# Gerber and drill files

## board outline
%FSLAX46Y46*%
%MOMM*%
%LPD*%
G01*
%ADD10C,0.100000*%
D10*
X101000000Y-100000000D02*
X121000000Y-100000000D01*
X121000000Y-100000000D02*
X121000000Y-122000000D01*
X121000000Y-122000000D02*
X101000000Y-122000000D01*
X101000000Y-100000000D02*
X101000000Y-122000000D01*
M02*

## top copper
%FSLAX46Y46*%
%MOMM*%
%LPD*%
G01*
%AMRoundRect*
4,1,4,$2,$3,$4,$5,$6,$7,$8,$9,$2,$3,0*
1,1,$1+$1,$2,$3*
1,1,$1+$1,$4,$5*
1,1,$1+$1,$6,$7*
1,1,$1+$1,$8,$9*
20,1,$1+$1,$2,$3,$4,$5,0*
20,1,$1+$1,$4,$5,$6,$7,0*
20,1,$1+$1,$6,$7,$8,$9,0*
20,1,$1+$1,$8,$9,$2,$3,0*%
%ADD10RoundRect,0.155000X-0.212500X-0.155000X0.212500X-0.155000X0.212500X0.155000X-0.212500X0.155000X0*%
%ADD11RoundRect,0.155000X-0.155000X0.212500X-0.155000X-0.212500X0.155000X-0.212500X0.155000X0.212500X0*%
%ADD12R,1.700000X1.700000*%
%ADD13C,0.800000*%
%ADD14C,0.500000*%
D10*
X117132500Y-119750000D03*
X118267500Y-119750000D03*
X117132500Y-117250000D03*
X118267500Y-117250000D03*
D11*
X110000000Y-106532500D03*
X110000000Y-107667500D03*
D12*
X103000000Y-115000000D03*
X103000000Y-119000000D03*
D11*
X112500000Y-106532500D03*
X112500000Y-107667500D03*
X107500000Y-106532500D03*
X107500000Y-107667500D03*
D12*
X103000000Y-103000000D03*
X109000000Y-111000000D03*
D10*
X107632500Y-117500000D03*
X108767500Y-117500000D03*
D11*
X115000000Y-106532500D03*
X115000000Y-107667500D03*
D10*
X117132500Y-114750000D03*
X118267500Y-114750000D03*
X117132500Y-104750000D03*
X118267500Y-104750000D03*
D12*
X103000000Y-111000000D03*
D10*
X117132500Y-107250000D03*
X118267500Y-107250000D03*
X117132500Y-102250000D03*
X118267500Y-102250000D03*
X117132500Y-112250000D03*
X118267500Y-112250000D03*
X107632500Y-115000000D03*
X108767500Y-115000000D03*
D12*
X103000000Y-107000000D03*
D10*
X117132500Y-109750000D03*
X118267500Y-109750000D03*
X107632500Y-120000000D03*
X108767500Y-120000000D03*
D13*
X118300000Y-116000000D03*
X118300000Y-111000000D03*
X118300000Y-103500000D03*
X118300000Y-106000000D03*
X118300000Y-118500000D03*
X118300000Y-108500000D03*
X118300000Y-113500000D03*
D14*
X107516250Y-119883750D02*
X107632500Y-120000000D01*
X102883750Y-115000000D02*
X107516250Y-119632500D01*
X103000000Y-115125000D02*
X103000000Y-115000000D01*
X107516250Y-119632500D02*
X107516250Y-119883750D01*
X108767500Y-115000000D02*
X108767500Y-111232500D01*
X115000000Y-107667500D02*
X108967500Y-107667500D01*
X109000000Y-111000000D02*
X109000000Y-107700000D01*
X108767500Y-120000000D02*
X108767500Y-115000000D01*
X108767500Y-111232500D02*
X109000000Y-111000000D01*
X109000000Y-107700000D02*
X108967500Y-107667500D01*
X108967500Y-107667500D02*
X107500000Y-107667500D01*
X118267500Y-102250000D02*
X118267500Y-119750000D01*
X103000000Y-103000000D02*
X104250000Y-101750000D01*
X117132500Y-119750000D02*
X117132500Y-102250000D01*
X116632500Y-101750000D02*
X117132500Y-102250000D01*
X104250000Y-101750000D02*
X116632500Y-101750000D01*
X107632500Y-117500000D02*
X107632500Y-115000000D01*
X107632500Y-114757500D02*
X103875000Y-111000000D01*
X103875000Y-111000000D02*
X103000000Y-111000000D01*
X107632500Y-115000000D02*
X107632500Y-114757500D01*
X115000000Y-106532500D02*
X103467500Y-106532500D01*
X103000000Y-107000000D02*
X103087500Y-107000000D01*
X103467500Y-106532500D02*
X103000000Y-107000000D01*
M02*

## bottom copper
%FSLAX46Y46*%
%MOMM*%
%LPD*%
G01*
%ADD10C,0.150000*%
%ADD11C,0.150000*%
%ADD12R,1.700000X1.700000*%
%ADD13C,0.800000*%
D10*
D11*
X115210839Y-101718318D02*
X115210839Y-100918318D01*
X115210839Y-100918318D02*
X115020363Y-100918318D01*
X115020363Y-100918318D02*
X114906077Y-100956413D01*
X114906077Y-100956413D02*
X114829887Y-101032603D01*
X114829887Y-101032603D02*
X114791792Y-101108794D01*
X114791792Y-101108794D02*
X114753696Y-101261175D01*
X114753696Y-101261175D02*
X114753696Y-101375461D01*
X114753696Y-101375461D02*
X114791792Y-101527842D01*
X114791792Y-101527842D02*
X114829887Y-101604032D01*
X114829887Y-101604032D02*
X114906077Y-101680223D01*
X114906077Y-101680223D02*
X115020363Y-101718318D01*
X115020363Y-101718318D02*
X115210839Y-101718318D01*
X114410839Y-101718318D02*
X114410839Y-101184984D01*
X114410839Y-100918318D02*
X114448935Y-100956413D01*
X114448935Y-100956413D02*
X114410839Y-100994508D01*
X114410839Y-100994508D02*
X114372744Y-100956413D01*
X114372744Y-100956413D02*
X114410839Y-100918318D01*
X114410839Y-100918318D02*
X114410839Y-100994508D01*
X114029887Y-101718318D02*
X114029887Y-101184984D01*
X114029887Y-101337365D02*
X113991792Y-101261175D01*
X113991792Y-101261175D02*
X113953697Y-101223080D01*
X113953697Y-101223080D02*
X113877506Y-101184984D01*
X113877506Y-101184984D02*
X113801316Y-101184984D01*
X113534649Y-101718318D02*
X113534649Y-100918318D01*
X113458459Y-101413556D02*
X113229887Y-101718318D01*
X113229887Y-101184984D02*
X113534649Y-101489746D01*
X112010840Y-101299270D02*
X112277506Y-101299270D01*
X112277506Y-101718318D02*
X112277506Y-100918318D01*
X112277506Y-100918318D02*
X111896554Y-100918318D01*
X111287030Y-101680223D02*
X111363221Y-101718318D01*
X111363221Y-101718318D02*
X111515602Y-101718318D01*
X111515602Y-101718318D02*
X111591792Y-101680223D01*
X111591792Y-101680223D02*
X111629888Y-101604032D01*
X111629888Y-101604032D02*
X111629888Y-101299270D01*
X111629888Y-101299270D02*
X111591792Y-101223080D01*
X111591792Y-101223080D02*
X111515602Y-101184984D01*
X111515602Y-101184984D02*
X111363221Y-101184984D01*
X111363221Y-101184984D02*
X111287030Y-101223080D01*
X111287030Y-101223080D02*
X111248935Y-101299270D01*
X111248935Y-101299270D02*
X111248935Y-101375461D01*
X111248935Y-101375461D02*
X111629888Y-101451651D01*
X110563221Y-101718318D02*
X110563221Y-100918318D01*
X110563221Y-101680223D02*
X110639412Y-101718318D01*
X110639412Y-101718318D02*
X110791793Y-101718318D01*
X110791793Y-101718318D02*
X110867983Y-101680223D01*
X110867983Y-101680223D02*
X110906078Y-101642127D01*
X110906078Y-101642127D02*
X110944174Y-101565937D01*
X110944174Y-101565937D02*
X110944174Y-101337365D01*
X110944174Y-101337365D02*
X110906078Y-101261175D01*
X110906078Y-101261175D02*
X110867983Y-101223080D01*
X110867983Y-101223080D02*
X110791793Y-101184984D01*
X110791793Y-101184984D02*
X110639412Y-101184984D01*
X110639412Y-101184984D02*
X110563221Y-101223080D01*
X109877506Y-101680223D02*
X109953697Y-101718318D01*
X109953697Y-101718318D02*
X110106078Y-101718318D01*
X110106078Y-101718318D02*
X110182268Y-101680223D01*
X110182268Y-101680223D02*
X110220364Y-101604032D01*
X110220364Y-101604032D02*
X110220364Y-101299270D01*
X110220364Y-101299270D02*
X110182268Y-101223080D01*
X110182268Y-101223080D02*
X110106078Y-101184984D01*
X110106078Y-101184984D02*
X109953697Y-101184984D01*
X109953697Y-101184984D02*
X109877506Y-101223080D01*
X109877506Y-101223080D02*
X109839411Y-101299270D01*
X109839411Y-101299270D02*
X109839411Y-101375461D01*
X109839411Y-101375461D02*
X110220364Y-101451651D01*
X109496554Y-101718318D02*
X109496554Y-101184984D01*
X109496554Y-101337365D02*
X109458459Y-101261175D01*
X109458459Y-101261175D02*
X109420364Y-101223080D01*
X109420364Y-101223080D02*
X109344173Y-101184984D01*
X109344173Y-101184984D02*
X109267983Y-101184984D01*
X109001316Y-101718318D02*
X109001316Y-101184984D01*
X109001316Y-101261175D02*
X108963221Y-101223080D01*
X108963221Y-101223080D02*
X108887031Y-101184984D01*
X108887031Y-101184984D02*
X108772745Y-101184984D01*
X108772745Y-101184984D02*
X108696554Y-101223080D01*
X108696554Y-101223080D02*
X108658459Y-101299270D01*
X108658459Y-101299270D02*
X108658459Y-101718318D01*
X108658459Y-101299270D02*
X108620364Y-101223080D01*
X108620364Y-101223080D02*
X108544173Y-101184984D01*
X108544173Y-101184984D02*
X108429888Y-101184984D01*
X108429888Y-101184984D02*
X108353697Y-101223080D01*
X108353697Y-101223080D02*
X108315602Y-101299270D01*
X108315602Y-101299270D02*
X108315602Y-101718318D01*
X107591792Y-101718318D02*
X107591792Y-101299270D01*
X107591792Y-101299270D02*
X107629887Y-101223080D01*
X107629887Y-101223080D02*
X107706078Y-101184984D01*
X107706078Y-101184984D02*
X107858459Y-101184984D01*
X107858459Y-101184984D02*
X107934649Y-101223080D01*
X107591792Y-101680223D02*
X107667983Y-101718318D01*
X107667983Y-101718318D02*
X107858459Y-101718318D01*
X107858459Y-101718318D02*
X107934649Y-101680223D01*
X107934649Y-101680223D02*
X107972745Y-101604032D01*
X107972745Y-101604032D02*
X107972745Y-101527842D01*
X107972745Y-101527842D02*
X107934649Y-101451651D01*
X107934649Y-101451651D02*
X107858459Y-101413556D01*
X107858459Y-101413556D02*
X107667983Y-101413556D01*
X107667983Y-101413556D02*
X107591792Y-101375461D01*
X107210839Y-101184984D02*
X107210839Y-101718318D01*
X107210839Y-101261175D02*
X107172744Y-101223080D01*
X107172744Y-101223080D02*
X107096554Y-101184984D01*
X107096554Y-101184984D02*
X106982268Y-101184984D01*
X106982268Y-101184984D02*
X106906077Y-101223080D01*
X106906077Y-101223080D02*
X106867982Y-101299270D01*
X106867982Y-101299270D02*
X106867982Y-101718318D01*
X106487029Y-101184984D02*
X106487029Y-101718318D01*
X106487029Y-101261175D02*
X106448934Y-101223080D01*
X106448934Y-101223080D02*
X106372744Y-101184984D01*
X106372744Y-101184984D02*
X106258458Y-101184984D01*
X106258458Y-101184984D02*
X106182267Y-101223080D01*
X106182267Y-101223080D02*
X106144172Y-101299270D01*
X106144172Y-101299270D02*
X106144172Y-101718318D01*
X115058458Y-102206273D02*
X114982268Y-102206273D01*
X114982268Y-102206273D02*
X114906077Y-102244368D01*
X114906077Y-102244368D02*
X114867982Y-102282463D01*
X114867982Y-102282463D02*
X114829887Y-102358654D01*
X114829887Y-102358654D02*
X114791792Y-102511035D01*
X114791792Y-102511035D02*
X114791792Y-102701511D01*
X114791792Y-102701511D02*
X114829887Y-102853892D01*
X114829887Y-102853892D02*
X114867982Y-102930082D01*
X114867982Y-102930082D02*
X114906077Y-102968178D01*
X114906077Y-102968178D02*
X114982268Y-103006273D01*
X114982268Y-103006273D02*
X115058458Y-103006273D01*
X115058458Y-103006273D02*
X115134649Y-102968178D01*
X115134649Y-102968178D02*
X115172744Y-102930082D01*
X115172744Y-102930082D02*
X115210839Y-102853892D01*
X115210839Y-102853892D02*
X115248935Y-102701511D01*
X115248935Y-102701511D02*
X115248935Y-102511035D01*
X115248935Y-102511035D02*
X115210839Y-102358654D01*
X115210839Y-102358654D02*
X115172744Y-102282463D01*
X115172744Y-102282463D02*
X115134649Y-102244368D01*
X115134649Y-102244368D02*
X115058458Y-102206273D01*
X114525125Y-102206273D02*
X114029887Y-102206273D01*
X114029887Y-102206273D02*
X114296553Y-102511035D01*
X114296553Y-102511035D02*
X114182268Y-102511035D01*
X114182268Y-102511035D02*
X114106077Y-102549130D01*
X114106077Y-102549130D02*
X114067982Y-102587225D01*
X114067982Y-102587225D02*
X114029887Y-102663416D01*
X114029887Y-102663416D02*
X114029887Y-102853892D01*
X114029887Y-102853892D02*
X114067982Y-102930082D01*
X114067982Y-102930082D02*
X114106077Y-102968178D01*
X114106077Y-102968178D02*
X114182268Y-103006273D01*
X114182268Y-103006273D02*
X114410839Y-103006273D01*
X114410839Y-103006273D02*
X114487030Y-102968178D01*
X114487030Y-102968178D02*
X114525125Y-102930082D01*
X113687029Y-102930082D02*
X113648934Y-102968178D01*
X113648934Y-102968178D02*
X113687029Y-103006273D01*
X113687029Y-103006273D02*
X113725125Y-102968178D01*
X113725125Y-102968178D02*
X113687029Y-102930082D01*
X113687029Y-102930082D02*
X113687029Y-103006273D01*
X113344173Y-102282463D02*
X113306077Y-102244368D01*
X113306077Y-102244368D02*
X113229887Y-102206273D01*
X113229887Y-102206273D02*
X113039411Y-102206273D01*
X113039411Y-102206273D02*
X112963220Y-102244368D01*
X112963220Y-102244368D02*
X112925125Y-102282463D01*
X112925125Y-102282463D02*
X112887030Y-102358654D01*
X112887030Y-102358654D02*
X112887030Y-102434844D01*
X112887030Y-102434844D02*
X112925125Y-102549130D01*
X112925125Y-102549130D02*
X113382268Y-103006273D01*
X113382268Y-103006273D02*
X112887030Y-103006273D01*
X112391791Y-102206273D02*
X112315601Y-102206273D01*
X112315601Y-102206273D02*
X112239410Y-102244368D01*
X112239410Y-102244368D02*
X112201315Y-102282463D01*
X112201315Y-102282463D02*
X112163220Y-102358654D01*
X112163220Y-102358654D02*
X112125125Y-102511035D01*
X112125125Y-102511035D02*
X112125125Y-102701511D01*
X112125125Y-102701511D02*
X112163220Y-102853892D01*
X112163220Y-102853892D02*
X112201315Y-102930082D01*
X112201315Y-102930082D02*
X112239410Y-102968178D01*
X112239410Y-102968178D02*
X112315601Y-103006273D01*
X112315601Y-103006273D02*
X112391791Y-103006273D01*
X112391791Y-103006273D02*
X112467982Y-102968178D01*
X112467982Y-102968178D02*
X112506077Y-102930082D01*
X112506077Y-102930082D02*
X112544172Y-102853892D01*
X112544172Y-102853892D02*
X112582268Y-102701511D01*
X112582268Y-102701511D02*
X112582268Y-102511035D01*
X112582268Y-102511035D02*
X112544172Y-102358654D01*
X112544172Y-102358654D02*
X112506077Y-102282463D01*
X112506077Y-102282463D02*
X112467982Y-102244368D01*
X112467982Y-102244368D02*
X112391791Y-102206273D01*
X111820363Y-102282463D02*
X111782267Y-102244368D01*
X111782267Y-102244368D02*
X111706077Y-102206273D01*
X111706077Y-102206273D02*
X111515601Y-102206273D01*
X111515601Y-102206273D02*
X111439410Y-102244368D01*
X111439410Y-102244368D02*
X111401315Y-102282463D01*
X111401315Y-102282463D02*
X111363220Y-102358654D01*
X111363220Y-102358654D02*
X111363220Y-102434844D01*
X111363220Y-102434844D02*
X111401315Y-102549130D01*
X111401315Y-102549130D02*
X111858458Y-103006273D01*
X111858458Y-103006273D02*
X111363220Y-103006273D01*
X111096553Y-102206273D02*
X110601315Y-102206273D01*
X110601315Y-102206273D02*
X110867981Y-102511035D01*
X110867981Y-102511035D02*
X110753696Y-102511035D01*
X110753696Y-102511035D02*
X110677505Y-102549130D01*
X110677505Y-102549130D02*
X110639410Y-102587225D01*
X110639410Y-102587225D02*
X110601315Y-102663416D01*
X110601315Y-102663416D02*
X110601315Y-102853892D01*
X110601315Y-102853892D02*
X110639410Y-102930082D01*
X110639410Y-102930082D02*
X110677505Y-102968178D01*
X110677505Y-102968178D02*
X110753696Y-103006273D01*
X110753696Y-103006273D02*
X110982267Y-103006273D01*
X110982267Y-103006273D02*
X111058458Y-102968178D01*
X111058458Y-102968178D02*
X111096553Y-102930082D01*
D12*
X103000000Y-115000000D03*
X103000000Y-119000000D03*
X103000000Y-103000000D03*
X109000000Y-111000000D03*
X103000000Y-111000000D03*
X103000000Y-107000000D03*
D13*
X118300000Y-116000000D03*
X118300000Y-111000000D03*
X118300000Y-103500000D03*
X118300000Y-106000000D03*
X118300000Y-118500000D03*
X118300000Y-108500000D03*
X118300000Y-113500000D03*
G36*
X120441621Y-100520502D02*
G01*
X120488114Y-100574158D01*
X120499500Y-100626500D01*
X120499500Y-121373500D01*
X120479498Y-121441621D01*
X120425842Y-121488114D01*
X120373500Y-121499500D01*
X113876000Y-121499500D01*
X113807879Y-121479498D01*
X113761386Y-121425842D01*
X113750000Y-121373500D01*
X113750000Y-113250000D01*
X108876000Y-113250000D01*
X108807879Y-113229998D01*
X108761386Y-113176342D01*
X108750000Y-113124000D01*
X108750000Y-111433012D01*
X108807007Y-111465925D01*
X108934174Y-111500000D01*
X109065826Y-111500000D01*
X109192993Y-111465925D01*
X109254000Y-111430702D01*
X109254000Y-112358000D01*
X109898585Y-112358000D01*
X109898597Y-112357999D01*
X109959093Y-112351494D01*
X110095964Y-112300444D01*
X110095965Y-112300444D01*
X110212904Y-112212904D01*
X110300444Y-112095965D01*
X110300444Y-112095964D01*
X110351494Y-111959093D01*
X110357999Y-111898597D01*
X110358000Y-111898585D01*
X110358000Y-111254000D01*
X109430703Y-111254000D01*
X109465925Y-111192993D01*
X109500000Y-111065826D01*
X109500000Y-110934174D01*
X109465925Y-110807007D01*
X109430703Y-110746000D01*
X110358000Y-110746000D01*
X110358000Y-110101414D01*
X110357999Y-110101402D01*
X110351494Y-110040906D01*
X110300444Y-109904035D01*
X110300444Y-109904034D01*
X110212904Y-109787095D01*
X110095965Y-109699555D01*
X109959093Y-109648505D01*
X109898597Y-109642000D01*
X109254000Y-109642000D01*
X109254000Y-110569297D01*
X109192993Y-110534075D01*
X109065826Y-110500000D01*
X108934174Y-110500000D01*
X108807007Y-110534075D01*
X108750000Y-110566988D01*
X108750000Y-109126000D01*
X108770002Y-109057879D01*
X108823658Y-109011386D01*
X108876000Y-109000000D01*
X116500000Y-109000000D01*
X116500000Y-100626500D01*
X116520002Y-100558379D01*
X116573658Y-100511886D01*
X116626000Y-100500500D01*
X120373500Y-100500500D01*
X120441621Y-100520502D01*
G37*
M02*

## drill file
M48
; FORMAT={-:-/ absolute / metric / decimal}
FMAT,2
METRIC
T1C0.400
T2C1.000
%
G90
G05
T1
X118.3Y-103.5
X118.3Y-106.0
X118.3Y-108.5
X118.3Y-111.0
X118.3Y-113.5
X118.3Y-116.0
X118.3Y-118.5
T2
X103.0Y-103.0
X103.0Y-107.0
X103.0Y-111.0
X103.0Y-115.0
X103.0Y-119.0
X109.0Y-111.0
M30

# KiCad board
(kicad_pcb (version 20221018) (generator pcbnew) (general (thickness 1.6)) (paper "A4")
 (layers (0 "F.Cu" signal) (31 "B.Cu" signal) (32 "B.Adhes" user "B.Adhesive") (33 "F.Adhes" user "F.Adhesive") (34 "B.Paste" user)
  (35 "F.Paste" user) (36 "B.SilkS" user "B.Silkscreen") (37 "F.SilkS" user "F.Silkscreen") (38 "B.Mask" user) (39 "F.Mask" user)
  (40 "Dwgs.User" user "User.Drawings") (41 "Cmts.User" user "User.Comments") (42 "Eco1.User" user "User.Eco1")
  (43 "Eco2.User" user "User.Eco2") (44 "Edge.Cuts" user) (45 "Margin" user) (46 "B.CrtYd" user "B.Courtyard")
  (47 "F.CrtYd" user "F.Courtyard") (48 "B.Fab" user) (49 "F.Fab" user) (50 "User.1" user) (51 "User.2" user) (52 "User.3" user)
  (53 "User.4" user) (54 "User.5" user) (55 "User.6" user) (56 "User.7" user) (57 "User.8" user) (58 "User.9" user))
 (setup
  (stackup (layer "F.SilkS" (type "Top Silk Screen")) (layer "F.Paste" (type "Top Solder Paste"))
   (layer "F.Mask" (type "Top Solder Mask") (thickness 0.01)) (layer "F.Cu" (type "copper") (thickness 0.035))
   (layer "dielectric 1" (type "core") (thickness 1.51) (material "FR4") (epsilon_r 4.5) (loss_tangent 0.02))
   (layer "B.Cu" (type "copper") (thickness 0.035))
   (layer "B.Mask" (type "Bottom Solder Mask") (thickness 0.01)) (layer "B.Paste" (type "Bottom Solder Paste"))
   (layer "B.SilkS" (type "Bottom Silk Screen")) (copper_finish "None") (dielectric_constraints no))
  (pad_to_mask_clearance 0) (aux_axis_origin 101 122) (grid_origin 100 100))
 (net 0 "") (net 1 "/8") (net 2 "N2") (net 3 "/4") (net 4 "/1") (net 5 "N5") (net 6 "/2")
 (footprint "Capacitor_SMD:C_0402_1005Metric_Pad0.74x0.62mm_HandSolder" (layer "F.Cu") (at 117.7 119.75)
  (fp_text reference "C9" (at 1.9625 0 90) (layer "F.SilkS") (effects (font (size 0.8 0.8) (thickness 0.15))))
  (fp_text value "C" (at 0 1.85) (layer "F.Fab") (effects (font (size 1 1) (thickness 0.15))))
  (pad "1" smd roundrect (at -0.5675 0) (size 0.735 0.62) (layers "F.Cu" "F.Paste" "F.Mask") (roundrect_rratio 0.25) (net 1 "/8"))
  (pad "2" smd roundrect (at 0.5675 0) (size 0.735 0.62) (layers "F.Cu" "F.Paste" "F.Mask") (roundrect_rratio 0.25) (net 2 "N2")))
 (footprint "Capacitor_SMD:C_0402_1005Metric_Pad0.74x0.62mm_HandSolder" (layer "F.Cu") (at 117.7 117.25)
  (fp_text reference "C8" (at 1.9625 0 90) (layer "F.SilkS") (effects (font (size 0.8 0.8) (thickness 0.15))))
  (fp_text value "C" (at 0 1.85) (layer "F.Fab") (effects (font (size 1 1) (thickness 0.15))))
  (pad "1" smd roundrect (at -0.5675 0) (size 0.735 0.62) (layers "F.Cu" "F.Paste" "F.Mask") (roundrect_rratio 0.25) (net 1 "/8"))
  (pad "2" smd roundrect (at 0.5675 0) (size 0.735 0.62) (layers "F.Cu" "F.Paste" "F.Mask") (roundrect_rratio 0.25) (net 2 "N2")))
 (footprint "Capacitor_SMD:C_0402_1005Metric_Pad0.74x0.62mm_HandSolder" (layer "F.Cu") (at 110 107.1 -90)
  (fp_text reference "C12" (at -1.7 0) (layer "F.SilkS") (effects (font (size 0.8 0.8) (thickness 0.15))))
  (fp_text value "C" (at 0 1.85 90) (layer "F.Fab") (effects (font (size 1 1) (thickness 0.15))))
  (pad "1" smd roundrect (at -0.5675 0 270) (size 0.735 0.62) (layers "F.Cu" "F.Paste" "F.Mask") (roundrect_rratio 0.25) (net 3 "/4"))
  (pad "2" smd roundrect (at 0.5675 0 270) (size 0.735 0.62) (layers "F.Cu" "F.Paste" "F.Mask") (roundrect_rratio 0.25) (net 2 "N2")))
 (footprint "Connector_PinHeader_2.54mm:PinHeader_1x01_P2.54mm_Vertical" (layer "F.Cu") (at 103 115)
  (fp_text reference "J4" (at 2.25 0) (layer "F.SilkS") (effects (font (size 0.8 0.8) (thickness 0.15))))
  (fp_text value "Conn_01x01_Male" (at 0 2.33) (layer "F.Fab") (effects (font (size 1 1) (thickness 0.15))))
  (pad "1" thru_hole rect (at 0 0) (size 1.7 1.7) (drill 1) (layers "*.Cu" "*.Mask") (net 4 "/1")))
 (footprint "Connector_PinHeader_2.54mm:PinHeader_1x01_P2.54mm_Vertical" (layer "F.Cu") (at 103 119)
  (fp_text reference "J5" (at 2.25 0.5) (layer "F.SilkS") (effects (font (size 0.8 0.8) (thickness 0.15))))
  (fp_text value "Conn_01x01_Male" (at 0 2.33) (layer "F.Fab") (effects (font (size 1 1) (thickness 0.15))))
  (pad "1" thru_hole rect (at 0 0) (size 1.7 1.7) (drill 1) (layers "*.Cu" "*.Mask") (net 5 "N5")))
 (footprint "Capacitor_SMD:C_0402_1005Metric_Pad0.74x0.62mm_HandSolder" (layer "F.Cu") (at 112.5 107.1 -90)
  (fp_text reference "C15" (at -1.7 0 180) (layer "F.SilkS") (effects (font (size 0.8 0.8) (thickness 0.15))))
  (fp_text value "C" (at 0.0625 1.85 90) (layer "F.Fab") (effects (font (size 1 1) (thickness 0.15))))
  (pad "1" smd roundrect (at -0.5675 0 270) (size 0.735 0.62) (layers "F.Cu" "F.Paste" "F.Mask") (roundrect_rratio 0.25) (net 3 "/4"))
  (pad "2" smd roundrect (at 0.5675 0 270) (size 0.735 0.62) (layers "F.Cu" "F.Paste" "F.Mask") (roundrect_rratio 0.25) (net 2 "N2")))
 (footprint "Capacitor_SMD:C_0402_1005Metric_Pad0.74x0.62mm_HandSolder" (layer "F.Cu") (at 107.5 107.1 -90)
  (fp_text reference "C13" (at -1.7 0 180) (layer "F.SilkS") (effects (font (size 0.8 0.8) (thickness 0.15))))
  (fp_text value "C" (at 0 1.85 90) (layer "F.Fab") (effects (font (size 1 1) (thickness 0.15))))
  (pad "1" smd roundrect (at -0.5675 0 270) (size 0.735 0.62) (layers "F.Cu" "F.Paste" "F.Mask") (roundrect_rratio 0.25) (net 3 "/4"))
  (pad "2" smd roundrect (at 0.5675 0 270) (size 0.735 0.62) (layers "F.Cu" "F.Paste" "F.Mask") (roundrect_rratio 0.25) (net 2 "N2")))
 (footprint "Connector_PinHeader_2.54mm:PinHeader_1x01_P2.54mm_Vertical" (layer "F.Cu") (at 103 103)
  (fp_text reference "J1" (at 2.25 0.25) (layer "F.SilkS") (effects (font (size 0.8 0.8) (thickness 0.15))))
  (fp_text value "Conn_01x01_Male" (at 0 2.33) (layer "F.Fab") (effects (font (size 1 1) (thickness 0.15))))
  (pad "1" thru_hole rect (at 0 0) (size 1.7 1.7) (drill 1) (layers "*.Cu" "*.Mask") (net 1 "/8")))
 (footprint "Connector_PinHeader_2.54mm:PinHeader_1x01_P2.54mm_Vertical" (layer "F.Cu") (at 109 111)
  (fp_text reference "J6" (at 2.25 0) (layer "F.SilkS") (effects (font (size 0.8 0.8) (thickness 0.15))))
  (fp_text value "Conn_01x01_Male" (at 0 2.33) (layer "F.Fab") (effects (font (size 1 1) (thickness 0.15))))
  (pad "1" thru_hole rect (at 0 0) (size 1.7 1.7) (drill 1) (layers "*.Cu" "*.Mask") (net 2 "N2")))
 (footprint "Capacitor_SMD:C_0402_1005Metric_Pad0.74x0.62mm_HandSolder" (layer "F.Cu") (at 108.2 117.5)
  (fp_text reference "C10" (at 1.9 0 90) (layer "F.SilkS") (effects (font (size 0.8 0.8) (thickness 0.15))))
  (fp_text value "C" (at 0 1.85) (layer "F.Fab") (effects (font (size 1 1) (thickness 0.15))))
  (pad "1" smd roundrect (at -0.5675 0) (size 0.735 0.62) (layers "F.Cu" "F.Paste" "F.Mask") (roundrect_rratio 0.25) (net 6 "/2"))
  (pad "2" smd roundrect (at 0.5675 0) (size 0.735 0.62) (layers "F.Cu" "F.Paste" "F.Mask") (roundrect_rratio 0.25) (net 2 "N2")))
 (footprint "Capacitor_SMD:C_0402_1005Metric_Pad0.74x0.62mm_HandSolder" (layer "F.Cu") (at 115 107.1 -90)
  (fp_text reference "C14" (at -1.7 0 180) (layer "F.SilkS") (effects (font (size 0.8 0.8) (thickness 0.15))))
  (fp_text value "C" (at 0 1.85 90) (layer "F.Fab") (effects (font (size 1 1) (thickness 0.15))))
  (pad "1" smd roundrect (at -0.5675 0 270) (size 0.735 0.62) (layers "F.Cu" "F.Paste" "F.Mask") (roundrect_rratio 0.25) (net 3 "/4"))
  (pad "2" smd roundrect (at 0.5675 0 270) (size 0.735 0.62) (layers "F.Cu" "F.Paste" "F.Mask") (roundrect_rratio 0.25) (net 2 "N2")))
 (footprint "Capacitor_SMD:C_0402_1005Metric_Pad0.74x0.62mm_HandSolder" (layer "F.Cu") (at 117.7 114.75)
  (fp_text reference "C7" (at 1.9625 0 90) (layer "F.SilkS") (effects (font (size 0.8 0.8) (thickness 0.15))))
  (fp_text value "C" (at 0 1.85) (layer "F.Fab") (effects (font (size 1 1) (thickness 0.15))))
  (pad "1" smd roundrect (at -0.5675 0) (size 0.735 0.62) (layers "F.Cu" "F.Paste" "F.Mask") (roundrect_rratio 0.25) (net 1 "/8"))
  (pad "2" smd roundrect (at 0.5675 0) (size 0.735 0.62) (layers "F.Cu" "F.Paste" "F.Mask") (roundrect_rratio 0.25) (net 2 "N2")))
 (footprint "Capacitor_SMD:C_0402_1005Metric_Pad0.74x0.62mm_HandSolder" (layer "F.Cu") (at 117.7 104.75)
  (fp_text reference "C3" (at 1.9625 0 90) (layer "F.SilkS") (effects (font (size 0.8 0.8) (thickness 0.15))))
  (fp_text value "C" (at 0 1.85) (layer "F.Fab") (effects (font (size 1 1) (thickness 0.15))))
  (pad "1" smd roundrect (at -0.5675 0) (size 0.735 0.62) (layers "F.Cu" "F.Paste" "F.Mask") (roundrect_rratio 0.25) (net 1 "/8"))
  (pad "2" smd roundrect (at 0.5675 0) (size 0.735 0.62) (layers "F.Cu" "F.Paste" "F.Mask") (roundrect_rratio 0.25) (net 2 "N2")))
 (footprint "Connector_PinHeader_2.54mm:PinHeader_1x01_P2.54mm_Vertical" (layer "F.Cu") (at 103 111)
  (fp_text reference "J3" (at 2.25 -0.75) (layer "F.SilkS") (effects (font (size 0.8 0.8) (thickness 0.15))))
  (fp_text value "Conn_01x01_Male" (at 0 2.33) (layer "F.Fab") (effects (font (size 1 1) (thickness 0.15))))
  (pad "1" thru_hole rect (at 0 0) (size 1.7 1.7) (drill 1) (layers "*.Cu" "*.Mask") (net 6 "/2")))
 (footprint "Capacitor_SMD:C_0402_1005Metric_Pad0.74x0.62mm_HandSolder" (layer "F.Cu") (at 117.7 107.25)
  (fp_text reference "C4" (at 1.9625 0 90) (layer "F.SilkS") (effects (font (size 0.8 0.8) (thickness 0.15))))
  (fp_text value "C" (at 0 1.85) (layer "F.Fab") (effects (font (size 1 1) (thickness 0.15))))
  (pad "1" smd roundrect (at -0.5675 0) (size 0.735 0.62) (layers "F.Cu" "F.Paste" "F.Mask") (roundrect_rratio 0.25) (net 1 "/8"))
  (pad "2" smd roundrect (at 0.5675 0) (size 0.735 0.62) (layers "F.Cu" "F.Paste" "F.Mask") (roundrect_rratio 0.25) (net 2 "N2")))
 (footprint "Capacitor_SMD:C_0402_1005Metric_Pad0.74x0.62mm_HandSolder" (layer "F.Cu") (at 117.7 102.25)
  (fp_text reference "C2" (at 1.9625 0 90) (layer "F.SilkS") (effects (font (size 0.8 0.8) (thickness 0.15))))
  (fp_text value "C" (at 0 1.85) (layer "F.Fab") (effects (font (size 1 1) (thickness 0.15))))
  (pad "1" smd roundrect (at -0.5675 0) (size 0.735 0.62) (layers "F.Cu" "F.Paste" "F.Mask") (roundrect_rratio 0.25) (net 1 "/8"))
  (pad "2" smd roundrect (at 0.5675 0) (size 0.735 0.62) (layers "F.Cu" "F.Paste" "F.Mask") (roundrect_rratio 0.25) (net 2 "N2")))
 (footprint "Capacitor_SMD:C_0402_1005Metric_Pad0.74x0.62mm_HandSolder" (layer "F.Cu") (at 117.7 112.25)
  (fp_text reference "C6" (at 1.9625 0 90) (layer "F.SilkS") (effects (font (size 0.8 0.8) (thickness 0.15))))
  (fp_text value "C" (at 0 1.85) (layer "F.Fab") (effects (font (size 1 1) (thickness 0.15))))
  (pad "1" smd roundrect (at -0.5675 0) (size 0.735 0.62) (layers "F.Cu" "F.Paste" "F.Mask") (roundrect_rratio 0.25) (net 1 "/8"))
  (pad "2" smd roundrect (at 0.5675 0) (size 0.735 0.62) (layers "F.Cu" "F.Paste" "F.Mask") (roundrect_rratio 0.25) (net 2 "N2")))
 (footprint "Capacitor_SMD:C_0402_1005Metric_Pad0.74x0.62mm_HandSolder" (layer "F.Cu") (at 108.2 115)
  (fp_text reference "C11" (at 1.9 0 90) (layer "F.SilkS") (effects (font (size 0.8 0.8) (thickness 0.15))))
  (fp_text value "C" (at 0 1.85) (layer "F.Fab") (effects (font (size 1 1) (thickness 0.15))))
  (pad "1" smd roundrect (at -0.5675 0) (size 0.735 0.62) (layers "F.Cu" "F.Paste" "F.Mask") (roundrect_rratio 0.25) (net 6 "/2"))
  (pad "2" smd roundrect (at 0.5675 0) (size 0.735 0.62) (layers "F.Cu" "F.Paste" "F.Mask") (roundrect_rratio 0.25) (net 2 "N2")))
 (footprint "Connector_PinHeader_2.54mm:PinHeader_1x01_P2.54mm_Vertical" (layer "F.Cu") (at 103 107)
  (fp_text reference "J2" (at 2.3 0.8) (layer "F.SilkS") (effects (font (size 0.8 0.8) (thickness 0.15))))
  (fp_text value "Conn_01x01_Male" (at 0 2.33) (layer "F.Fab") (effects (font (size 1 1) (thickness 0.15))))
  (pad "1" thru_hole rect (at 0 0) (size 1.7 1.7) (drill 1) (layers "*.Cu" "*.Mask") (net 3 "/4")))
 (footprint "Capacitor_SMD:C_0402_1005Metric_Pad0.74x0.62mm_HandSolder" (layer "F.Cu") (at 117.7 109.75)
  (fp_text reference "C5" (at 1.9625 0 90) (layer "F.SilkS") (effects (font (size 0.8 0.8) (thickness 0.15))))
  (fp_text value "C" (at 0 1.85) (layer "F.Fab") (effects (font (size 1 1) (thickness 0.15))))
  (pad "1" smd roundrect (at -0.5675 0) (size 0.735 0.62) (layers "F.Cu" "F.Paste" "F.Mask") (roundrect_rratio 0.25) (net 1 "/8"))
  (pad "2" smd roundrect (at 0.5675 0) (size 0.735 0.62) (layers "F.Cu" "F.Paste" "F.Mask") (roundrect_rratio 0.25) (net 2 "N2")))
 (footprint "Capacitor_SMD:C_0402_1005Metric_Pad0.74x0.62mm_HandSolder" (layer "F.Cu") (at 108.2 120)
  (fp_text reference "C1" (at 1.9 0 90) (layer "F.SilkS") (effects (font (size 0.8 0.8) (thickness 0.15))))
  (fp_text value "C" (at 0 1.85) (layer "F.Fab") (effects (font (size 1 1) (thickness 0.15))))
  (pad "1" smd roundrect (at -0.5675 0) (size 0.735 0.62) (layers "F.Cu" "F.Paste" "F.Mask") (roundrect_rratio 0.25) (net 4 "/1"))
  (pad "2" smd roundrect (at 0.5675 0) (size 0.735 0.62) (layers "F.Cu" "F.Paste" "F.Mask") (roundrect_rratio 0.25) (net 2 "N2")))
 (gr_line (start 101 100) (end 121 100) (stroke (width 0.1) (type solid)) (layer "Edge.Cuts"))
 (gr_line (start 121 100) (end 121 122) (stroke (width 0.1) (type solid)) (layer "Edge.Cuts"))
 (gr_line (start 121 122) (end 101 122) (stroke (width 0.1) (type solid)) (layer "Edge.Cuts"))
 (gr_line (start 101 100) (end 101 122) (stroke (width 0.1) (type solid)) (layer "Edge.Cuts"))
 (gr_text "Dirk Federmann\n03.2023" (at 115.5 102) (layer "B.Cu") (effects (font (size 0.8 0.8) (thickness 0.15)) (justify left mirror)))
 (segment (start 107.51625 119.88375) (end 107.6325 120) (width 0.5) (layer "F.Cu") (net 4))
 (segment (start 102.88375 115) (end 107.51625 119.6325) (width 0.5) (layer "F.Cu") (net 4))
 (segment (start 103 115.125) (end 103 115) (width 0.5) (layer "F.Cu") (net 4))
 (segment (start 107.51625 119.6325) (end 107.51625 119.88375) (width 0.5) (layer "F.Cu") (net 4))
 (segment (start 108.7675 115) (end 108.7675 111.2325) (width 0.5) (layer "F.Cu") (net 2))
 (segment (start 115 107.6675) (end 108.9675 107.6675) (width 0.5) (layer "F.Cu") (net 2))
 (segment (start 109 111) (end 109 107.7) (width 0.5) (layer "F.Cu") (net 2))
 (segment (start 108.7675 120) (end 108.7675 115) (width 0.5) (layer "F.Cu") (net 2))
 (segment (start 108.7675 111.2325) (end 109 111) (width 0.5) (layer "F.Cu") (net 2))
 (segment (start 109 107.7) (end 108.9675 107.6675) (width 0.5) (layer "F.Cu") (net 2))
 (segment (start 108.9675 107.6675) (end 107.5 107.6675) (width 0.5) (layer "F.Cu") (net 2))
 (segment (start 118.2675 102.25) (end 118.2675 119.75) (width 0.5) (layer "F.Cu") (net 2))
 (via (at 118.3 116) (size 0.8) (drill 0.4) (layers "F.Cu" "B.Cu") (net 2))
 (via (at 118.3 111) (size 0.8) (drill 0.4) (layers "F.Cu" "B.Cu") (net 2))
 (via (at 118.3 103.5) (size 0.8) (drill 0.4) (layers "F.Cu" "B.Cu") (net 2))
 (via (at 118.3 106) (size 0.8) (drill 0.4) (layers "F.Cu" "B.Cu") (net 2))
 (via (at 118.3 118.5) (size 0.8) (drill 0.4) (layers "F.Cu" "B.Cu") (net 2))
 (via (at 118.3 108.5) (size 0.8) (drill 0.4) (layers "F.Cu" "B.Cu") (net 2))
 (via (at 118.3 113.5) (size 0.8) (drill 0.4) (layers "F.Cu" "B.Cu") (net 2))
 (segment (start 103 103) (end 104.25 101.75) (width 0.5) (layer "F.Cu") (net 1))
 (segment (start 117.1325 119.75) (end 117.1325 102.25) (width 0.5) (layer "F.Cu") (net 1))
 (segment (start 116.6325 101.75) (end 117.1325 102.25) (width 0.5) (layer "F.Cu") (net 1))
 (segment (start 104.25 101.75) (end 116.6325 101.75) (width 0.5) (layer "F.Cu") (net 1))
 (segment (start 107.6325 117.5) (end 107.6325 115) (width 0.5) (layer "F.Cu") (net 6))
 (segment (start 107.6325 114.7575) (end 103.875 111) (width 0.5) (layer "F.Cu") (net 6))
 (segment (start 103.875 111) (end 103 111) (width 0.5) (layer "F.Cu") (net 6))
 (segment (start 107.6325 115) (end 107.6325 114.7575) (width 0.5) (layer "F.Cu") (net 6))
 (segment (start 115 106.5325) (end 103.4675 106.5325) (width 0.5) (layer "F.Cu") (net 3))
 (segment (start 103 107) (end 103.0875 107) (width 0.5) (layer "F.Cu") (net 3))
 (segment (start 103.4675 106.5325) (end 103 107) (width 0.5) (layer "F.Cu") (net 3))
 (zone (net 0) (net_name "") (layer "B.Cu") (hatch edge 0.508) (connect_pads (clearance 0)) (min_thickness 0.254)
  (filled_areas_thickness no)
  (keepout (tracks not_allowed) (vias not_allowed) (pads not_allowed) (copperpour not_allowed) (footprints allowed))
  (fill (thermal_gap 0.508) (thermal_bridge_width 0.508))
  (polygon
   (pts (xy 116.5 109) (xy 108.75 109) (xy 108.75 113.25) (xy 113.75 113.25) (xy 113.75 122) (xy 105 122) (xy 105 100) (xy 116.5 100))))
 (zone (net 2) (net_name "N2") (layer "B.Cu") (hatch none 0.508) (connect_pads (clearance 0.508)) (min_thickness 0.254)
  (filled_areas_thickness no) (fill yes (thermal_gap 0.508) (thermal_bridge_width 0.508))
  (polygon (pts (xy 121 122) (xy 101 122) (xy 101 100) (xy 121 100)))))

